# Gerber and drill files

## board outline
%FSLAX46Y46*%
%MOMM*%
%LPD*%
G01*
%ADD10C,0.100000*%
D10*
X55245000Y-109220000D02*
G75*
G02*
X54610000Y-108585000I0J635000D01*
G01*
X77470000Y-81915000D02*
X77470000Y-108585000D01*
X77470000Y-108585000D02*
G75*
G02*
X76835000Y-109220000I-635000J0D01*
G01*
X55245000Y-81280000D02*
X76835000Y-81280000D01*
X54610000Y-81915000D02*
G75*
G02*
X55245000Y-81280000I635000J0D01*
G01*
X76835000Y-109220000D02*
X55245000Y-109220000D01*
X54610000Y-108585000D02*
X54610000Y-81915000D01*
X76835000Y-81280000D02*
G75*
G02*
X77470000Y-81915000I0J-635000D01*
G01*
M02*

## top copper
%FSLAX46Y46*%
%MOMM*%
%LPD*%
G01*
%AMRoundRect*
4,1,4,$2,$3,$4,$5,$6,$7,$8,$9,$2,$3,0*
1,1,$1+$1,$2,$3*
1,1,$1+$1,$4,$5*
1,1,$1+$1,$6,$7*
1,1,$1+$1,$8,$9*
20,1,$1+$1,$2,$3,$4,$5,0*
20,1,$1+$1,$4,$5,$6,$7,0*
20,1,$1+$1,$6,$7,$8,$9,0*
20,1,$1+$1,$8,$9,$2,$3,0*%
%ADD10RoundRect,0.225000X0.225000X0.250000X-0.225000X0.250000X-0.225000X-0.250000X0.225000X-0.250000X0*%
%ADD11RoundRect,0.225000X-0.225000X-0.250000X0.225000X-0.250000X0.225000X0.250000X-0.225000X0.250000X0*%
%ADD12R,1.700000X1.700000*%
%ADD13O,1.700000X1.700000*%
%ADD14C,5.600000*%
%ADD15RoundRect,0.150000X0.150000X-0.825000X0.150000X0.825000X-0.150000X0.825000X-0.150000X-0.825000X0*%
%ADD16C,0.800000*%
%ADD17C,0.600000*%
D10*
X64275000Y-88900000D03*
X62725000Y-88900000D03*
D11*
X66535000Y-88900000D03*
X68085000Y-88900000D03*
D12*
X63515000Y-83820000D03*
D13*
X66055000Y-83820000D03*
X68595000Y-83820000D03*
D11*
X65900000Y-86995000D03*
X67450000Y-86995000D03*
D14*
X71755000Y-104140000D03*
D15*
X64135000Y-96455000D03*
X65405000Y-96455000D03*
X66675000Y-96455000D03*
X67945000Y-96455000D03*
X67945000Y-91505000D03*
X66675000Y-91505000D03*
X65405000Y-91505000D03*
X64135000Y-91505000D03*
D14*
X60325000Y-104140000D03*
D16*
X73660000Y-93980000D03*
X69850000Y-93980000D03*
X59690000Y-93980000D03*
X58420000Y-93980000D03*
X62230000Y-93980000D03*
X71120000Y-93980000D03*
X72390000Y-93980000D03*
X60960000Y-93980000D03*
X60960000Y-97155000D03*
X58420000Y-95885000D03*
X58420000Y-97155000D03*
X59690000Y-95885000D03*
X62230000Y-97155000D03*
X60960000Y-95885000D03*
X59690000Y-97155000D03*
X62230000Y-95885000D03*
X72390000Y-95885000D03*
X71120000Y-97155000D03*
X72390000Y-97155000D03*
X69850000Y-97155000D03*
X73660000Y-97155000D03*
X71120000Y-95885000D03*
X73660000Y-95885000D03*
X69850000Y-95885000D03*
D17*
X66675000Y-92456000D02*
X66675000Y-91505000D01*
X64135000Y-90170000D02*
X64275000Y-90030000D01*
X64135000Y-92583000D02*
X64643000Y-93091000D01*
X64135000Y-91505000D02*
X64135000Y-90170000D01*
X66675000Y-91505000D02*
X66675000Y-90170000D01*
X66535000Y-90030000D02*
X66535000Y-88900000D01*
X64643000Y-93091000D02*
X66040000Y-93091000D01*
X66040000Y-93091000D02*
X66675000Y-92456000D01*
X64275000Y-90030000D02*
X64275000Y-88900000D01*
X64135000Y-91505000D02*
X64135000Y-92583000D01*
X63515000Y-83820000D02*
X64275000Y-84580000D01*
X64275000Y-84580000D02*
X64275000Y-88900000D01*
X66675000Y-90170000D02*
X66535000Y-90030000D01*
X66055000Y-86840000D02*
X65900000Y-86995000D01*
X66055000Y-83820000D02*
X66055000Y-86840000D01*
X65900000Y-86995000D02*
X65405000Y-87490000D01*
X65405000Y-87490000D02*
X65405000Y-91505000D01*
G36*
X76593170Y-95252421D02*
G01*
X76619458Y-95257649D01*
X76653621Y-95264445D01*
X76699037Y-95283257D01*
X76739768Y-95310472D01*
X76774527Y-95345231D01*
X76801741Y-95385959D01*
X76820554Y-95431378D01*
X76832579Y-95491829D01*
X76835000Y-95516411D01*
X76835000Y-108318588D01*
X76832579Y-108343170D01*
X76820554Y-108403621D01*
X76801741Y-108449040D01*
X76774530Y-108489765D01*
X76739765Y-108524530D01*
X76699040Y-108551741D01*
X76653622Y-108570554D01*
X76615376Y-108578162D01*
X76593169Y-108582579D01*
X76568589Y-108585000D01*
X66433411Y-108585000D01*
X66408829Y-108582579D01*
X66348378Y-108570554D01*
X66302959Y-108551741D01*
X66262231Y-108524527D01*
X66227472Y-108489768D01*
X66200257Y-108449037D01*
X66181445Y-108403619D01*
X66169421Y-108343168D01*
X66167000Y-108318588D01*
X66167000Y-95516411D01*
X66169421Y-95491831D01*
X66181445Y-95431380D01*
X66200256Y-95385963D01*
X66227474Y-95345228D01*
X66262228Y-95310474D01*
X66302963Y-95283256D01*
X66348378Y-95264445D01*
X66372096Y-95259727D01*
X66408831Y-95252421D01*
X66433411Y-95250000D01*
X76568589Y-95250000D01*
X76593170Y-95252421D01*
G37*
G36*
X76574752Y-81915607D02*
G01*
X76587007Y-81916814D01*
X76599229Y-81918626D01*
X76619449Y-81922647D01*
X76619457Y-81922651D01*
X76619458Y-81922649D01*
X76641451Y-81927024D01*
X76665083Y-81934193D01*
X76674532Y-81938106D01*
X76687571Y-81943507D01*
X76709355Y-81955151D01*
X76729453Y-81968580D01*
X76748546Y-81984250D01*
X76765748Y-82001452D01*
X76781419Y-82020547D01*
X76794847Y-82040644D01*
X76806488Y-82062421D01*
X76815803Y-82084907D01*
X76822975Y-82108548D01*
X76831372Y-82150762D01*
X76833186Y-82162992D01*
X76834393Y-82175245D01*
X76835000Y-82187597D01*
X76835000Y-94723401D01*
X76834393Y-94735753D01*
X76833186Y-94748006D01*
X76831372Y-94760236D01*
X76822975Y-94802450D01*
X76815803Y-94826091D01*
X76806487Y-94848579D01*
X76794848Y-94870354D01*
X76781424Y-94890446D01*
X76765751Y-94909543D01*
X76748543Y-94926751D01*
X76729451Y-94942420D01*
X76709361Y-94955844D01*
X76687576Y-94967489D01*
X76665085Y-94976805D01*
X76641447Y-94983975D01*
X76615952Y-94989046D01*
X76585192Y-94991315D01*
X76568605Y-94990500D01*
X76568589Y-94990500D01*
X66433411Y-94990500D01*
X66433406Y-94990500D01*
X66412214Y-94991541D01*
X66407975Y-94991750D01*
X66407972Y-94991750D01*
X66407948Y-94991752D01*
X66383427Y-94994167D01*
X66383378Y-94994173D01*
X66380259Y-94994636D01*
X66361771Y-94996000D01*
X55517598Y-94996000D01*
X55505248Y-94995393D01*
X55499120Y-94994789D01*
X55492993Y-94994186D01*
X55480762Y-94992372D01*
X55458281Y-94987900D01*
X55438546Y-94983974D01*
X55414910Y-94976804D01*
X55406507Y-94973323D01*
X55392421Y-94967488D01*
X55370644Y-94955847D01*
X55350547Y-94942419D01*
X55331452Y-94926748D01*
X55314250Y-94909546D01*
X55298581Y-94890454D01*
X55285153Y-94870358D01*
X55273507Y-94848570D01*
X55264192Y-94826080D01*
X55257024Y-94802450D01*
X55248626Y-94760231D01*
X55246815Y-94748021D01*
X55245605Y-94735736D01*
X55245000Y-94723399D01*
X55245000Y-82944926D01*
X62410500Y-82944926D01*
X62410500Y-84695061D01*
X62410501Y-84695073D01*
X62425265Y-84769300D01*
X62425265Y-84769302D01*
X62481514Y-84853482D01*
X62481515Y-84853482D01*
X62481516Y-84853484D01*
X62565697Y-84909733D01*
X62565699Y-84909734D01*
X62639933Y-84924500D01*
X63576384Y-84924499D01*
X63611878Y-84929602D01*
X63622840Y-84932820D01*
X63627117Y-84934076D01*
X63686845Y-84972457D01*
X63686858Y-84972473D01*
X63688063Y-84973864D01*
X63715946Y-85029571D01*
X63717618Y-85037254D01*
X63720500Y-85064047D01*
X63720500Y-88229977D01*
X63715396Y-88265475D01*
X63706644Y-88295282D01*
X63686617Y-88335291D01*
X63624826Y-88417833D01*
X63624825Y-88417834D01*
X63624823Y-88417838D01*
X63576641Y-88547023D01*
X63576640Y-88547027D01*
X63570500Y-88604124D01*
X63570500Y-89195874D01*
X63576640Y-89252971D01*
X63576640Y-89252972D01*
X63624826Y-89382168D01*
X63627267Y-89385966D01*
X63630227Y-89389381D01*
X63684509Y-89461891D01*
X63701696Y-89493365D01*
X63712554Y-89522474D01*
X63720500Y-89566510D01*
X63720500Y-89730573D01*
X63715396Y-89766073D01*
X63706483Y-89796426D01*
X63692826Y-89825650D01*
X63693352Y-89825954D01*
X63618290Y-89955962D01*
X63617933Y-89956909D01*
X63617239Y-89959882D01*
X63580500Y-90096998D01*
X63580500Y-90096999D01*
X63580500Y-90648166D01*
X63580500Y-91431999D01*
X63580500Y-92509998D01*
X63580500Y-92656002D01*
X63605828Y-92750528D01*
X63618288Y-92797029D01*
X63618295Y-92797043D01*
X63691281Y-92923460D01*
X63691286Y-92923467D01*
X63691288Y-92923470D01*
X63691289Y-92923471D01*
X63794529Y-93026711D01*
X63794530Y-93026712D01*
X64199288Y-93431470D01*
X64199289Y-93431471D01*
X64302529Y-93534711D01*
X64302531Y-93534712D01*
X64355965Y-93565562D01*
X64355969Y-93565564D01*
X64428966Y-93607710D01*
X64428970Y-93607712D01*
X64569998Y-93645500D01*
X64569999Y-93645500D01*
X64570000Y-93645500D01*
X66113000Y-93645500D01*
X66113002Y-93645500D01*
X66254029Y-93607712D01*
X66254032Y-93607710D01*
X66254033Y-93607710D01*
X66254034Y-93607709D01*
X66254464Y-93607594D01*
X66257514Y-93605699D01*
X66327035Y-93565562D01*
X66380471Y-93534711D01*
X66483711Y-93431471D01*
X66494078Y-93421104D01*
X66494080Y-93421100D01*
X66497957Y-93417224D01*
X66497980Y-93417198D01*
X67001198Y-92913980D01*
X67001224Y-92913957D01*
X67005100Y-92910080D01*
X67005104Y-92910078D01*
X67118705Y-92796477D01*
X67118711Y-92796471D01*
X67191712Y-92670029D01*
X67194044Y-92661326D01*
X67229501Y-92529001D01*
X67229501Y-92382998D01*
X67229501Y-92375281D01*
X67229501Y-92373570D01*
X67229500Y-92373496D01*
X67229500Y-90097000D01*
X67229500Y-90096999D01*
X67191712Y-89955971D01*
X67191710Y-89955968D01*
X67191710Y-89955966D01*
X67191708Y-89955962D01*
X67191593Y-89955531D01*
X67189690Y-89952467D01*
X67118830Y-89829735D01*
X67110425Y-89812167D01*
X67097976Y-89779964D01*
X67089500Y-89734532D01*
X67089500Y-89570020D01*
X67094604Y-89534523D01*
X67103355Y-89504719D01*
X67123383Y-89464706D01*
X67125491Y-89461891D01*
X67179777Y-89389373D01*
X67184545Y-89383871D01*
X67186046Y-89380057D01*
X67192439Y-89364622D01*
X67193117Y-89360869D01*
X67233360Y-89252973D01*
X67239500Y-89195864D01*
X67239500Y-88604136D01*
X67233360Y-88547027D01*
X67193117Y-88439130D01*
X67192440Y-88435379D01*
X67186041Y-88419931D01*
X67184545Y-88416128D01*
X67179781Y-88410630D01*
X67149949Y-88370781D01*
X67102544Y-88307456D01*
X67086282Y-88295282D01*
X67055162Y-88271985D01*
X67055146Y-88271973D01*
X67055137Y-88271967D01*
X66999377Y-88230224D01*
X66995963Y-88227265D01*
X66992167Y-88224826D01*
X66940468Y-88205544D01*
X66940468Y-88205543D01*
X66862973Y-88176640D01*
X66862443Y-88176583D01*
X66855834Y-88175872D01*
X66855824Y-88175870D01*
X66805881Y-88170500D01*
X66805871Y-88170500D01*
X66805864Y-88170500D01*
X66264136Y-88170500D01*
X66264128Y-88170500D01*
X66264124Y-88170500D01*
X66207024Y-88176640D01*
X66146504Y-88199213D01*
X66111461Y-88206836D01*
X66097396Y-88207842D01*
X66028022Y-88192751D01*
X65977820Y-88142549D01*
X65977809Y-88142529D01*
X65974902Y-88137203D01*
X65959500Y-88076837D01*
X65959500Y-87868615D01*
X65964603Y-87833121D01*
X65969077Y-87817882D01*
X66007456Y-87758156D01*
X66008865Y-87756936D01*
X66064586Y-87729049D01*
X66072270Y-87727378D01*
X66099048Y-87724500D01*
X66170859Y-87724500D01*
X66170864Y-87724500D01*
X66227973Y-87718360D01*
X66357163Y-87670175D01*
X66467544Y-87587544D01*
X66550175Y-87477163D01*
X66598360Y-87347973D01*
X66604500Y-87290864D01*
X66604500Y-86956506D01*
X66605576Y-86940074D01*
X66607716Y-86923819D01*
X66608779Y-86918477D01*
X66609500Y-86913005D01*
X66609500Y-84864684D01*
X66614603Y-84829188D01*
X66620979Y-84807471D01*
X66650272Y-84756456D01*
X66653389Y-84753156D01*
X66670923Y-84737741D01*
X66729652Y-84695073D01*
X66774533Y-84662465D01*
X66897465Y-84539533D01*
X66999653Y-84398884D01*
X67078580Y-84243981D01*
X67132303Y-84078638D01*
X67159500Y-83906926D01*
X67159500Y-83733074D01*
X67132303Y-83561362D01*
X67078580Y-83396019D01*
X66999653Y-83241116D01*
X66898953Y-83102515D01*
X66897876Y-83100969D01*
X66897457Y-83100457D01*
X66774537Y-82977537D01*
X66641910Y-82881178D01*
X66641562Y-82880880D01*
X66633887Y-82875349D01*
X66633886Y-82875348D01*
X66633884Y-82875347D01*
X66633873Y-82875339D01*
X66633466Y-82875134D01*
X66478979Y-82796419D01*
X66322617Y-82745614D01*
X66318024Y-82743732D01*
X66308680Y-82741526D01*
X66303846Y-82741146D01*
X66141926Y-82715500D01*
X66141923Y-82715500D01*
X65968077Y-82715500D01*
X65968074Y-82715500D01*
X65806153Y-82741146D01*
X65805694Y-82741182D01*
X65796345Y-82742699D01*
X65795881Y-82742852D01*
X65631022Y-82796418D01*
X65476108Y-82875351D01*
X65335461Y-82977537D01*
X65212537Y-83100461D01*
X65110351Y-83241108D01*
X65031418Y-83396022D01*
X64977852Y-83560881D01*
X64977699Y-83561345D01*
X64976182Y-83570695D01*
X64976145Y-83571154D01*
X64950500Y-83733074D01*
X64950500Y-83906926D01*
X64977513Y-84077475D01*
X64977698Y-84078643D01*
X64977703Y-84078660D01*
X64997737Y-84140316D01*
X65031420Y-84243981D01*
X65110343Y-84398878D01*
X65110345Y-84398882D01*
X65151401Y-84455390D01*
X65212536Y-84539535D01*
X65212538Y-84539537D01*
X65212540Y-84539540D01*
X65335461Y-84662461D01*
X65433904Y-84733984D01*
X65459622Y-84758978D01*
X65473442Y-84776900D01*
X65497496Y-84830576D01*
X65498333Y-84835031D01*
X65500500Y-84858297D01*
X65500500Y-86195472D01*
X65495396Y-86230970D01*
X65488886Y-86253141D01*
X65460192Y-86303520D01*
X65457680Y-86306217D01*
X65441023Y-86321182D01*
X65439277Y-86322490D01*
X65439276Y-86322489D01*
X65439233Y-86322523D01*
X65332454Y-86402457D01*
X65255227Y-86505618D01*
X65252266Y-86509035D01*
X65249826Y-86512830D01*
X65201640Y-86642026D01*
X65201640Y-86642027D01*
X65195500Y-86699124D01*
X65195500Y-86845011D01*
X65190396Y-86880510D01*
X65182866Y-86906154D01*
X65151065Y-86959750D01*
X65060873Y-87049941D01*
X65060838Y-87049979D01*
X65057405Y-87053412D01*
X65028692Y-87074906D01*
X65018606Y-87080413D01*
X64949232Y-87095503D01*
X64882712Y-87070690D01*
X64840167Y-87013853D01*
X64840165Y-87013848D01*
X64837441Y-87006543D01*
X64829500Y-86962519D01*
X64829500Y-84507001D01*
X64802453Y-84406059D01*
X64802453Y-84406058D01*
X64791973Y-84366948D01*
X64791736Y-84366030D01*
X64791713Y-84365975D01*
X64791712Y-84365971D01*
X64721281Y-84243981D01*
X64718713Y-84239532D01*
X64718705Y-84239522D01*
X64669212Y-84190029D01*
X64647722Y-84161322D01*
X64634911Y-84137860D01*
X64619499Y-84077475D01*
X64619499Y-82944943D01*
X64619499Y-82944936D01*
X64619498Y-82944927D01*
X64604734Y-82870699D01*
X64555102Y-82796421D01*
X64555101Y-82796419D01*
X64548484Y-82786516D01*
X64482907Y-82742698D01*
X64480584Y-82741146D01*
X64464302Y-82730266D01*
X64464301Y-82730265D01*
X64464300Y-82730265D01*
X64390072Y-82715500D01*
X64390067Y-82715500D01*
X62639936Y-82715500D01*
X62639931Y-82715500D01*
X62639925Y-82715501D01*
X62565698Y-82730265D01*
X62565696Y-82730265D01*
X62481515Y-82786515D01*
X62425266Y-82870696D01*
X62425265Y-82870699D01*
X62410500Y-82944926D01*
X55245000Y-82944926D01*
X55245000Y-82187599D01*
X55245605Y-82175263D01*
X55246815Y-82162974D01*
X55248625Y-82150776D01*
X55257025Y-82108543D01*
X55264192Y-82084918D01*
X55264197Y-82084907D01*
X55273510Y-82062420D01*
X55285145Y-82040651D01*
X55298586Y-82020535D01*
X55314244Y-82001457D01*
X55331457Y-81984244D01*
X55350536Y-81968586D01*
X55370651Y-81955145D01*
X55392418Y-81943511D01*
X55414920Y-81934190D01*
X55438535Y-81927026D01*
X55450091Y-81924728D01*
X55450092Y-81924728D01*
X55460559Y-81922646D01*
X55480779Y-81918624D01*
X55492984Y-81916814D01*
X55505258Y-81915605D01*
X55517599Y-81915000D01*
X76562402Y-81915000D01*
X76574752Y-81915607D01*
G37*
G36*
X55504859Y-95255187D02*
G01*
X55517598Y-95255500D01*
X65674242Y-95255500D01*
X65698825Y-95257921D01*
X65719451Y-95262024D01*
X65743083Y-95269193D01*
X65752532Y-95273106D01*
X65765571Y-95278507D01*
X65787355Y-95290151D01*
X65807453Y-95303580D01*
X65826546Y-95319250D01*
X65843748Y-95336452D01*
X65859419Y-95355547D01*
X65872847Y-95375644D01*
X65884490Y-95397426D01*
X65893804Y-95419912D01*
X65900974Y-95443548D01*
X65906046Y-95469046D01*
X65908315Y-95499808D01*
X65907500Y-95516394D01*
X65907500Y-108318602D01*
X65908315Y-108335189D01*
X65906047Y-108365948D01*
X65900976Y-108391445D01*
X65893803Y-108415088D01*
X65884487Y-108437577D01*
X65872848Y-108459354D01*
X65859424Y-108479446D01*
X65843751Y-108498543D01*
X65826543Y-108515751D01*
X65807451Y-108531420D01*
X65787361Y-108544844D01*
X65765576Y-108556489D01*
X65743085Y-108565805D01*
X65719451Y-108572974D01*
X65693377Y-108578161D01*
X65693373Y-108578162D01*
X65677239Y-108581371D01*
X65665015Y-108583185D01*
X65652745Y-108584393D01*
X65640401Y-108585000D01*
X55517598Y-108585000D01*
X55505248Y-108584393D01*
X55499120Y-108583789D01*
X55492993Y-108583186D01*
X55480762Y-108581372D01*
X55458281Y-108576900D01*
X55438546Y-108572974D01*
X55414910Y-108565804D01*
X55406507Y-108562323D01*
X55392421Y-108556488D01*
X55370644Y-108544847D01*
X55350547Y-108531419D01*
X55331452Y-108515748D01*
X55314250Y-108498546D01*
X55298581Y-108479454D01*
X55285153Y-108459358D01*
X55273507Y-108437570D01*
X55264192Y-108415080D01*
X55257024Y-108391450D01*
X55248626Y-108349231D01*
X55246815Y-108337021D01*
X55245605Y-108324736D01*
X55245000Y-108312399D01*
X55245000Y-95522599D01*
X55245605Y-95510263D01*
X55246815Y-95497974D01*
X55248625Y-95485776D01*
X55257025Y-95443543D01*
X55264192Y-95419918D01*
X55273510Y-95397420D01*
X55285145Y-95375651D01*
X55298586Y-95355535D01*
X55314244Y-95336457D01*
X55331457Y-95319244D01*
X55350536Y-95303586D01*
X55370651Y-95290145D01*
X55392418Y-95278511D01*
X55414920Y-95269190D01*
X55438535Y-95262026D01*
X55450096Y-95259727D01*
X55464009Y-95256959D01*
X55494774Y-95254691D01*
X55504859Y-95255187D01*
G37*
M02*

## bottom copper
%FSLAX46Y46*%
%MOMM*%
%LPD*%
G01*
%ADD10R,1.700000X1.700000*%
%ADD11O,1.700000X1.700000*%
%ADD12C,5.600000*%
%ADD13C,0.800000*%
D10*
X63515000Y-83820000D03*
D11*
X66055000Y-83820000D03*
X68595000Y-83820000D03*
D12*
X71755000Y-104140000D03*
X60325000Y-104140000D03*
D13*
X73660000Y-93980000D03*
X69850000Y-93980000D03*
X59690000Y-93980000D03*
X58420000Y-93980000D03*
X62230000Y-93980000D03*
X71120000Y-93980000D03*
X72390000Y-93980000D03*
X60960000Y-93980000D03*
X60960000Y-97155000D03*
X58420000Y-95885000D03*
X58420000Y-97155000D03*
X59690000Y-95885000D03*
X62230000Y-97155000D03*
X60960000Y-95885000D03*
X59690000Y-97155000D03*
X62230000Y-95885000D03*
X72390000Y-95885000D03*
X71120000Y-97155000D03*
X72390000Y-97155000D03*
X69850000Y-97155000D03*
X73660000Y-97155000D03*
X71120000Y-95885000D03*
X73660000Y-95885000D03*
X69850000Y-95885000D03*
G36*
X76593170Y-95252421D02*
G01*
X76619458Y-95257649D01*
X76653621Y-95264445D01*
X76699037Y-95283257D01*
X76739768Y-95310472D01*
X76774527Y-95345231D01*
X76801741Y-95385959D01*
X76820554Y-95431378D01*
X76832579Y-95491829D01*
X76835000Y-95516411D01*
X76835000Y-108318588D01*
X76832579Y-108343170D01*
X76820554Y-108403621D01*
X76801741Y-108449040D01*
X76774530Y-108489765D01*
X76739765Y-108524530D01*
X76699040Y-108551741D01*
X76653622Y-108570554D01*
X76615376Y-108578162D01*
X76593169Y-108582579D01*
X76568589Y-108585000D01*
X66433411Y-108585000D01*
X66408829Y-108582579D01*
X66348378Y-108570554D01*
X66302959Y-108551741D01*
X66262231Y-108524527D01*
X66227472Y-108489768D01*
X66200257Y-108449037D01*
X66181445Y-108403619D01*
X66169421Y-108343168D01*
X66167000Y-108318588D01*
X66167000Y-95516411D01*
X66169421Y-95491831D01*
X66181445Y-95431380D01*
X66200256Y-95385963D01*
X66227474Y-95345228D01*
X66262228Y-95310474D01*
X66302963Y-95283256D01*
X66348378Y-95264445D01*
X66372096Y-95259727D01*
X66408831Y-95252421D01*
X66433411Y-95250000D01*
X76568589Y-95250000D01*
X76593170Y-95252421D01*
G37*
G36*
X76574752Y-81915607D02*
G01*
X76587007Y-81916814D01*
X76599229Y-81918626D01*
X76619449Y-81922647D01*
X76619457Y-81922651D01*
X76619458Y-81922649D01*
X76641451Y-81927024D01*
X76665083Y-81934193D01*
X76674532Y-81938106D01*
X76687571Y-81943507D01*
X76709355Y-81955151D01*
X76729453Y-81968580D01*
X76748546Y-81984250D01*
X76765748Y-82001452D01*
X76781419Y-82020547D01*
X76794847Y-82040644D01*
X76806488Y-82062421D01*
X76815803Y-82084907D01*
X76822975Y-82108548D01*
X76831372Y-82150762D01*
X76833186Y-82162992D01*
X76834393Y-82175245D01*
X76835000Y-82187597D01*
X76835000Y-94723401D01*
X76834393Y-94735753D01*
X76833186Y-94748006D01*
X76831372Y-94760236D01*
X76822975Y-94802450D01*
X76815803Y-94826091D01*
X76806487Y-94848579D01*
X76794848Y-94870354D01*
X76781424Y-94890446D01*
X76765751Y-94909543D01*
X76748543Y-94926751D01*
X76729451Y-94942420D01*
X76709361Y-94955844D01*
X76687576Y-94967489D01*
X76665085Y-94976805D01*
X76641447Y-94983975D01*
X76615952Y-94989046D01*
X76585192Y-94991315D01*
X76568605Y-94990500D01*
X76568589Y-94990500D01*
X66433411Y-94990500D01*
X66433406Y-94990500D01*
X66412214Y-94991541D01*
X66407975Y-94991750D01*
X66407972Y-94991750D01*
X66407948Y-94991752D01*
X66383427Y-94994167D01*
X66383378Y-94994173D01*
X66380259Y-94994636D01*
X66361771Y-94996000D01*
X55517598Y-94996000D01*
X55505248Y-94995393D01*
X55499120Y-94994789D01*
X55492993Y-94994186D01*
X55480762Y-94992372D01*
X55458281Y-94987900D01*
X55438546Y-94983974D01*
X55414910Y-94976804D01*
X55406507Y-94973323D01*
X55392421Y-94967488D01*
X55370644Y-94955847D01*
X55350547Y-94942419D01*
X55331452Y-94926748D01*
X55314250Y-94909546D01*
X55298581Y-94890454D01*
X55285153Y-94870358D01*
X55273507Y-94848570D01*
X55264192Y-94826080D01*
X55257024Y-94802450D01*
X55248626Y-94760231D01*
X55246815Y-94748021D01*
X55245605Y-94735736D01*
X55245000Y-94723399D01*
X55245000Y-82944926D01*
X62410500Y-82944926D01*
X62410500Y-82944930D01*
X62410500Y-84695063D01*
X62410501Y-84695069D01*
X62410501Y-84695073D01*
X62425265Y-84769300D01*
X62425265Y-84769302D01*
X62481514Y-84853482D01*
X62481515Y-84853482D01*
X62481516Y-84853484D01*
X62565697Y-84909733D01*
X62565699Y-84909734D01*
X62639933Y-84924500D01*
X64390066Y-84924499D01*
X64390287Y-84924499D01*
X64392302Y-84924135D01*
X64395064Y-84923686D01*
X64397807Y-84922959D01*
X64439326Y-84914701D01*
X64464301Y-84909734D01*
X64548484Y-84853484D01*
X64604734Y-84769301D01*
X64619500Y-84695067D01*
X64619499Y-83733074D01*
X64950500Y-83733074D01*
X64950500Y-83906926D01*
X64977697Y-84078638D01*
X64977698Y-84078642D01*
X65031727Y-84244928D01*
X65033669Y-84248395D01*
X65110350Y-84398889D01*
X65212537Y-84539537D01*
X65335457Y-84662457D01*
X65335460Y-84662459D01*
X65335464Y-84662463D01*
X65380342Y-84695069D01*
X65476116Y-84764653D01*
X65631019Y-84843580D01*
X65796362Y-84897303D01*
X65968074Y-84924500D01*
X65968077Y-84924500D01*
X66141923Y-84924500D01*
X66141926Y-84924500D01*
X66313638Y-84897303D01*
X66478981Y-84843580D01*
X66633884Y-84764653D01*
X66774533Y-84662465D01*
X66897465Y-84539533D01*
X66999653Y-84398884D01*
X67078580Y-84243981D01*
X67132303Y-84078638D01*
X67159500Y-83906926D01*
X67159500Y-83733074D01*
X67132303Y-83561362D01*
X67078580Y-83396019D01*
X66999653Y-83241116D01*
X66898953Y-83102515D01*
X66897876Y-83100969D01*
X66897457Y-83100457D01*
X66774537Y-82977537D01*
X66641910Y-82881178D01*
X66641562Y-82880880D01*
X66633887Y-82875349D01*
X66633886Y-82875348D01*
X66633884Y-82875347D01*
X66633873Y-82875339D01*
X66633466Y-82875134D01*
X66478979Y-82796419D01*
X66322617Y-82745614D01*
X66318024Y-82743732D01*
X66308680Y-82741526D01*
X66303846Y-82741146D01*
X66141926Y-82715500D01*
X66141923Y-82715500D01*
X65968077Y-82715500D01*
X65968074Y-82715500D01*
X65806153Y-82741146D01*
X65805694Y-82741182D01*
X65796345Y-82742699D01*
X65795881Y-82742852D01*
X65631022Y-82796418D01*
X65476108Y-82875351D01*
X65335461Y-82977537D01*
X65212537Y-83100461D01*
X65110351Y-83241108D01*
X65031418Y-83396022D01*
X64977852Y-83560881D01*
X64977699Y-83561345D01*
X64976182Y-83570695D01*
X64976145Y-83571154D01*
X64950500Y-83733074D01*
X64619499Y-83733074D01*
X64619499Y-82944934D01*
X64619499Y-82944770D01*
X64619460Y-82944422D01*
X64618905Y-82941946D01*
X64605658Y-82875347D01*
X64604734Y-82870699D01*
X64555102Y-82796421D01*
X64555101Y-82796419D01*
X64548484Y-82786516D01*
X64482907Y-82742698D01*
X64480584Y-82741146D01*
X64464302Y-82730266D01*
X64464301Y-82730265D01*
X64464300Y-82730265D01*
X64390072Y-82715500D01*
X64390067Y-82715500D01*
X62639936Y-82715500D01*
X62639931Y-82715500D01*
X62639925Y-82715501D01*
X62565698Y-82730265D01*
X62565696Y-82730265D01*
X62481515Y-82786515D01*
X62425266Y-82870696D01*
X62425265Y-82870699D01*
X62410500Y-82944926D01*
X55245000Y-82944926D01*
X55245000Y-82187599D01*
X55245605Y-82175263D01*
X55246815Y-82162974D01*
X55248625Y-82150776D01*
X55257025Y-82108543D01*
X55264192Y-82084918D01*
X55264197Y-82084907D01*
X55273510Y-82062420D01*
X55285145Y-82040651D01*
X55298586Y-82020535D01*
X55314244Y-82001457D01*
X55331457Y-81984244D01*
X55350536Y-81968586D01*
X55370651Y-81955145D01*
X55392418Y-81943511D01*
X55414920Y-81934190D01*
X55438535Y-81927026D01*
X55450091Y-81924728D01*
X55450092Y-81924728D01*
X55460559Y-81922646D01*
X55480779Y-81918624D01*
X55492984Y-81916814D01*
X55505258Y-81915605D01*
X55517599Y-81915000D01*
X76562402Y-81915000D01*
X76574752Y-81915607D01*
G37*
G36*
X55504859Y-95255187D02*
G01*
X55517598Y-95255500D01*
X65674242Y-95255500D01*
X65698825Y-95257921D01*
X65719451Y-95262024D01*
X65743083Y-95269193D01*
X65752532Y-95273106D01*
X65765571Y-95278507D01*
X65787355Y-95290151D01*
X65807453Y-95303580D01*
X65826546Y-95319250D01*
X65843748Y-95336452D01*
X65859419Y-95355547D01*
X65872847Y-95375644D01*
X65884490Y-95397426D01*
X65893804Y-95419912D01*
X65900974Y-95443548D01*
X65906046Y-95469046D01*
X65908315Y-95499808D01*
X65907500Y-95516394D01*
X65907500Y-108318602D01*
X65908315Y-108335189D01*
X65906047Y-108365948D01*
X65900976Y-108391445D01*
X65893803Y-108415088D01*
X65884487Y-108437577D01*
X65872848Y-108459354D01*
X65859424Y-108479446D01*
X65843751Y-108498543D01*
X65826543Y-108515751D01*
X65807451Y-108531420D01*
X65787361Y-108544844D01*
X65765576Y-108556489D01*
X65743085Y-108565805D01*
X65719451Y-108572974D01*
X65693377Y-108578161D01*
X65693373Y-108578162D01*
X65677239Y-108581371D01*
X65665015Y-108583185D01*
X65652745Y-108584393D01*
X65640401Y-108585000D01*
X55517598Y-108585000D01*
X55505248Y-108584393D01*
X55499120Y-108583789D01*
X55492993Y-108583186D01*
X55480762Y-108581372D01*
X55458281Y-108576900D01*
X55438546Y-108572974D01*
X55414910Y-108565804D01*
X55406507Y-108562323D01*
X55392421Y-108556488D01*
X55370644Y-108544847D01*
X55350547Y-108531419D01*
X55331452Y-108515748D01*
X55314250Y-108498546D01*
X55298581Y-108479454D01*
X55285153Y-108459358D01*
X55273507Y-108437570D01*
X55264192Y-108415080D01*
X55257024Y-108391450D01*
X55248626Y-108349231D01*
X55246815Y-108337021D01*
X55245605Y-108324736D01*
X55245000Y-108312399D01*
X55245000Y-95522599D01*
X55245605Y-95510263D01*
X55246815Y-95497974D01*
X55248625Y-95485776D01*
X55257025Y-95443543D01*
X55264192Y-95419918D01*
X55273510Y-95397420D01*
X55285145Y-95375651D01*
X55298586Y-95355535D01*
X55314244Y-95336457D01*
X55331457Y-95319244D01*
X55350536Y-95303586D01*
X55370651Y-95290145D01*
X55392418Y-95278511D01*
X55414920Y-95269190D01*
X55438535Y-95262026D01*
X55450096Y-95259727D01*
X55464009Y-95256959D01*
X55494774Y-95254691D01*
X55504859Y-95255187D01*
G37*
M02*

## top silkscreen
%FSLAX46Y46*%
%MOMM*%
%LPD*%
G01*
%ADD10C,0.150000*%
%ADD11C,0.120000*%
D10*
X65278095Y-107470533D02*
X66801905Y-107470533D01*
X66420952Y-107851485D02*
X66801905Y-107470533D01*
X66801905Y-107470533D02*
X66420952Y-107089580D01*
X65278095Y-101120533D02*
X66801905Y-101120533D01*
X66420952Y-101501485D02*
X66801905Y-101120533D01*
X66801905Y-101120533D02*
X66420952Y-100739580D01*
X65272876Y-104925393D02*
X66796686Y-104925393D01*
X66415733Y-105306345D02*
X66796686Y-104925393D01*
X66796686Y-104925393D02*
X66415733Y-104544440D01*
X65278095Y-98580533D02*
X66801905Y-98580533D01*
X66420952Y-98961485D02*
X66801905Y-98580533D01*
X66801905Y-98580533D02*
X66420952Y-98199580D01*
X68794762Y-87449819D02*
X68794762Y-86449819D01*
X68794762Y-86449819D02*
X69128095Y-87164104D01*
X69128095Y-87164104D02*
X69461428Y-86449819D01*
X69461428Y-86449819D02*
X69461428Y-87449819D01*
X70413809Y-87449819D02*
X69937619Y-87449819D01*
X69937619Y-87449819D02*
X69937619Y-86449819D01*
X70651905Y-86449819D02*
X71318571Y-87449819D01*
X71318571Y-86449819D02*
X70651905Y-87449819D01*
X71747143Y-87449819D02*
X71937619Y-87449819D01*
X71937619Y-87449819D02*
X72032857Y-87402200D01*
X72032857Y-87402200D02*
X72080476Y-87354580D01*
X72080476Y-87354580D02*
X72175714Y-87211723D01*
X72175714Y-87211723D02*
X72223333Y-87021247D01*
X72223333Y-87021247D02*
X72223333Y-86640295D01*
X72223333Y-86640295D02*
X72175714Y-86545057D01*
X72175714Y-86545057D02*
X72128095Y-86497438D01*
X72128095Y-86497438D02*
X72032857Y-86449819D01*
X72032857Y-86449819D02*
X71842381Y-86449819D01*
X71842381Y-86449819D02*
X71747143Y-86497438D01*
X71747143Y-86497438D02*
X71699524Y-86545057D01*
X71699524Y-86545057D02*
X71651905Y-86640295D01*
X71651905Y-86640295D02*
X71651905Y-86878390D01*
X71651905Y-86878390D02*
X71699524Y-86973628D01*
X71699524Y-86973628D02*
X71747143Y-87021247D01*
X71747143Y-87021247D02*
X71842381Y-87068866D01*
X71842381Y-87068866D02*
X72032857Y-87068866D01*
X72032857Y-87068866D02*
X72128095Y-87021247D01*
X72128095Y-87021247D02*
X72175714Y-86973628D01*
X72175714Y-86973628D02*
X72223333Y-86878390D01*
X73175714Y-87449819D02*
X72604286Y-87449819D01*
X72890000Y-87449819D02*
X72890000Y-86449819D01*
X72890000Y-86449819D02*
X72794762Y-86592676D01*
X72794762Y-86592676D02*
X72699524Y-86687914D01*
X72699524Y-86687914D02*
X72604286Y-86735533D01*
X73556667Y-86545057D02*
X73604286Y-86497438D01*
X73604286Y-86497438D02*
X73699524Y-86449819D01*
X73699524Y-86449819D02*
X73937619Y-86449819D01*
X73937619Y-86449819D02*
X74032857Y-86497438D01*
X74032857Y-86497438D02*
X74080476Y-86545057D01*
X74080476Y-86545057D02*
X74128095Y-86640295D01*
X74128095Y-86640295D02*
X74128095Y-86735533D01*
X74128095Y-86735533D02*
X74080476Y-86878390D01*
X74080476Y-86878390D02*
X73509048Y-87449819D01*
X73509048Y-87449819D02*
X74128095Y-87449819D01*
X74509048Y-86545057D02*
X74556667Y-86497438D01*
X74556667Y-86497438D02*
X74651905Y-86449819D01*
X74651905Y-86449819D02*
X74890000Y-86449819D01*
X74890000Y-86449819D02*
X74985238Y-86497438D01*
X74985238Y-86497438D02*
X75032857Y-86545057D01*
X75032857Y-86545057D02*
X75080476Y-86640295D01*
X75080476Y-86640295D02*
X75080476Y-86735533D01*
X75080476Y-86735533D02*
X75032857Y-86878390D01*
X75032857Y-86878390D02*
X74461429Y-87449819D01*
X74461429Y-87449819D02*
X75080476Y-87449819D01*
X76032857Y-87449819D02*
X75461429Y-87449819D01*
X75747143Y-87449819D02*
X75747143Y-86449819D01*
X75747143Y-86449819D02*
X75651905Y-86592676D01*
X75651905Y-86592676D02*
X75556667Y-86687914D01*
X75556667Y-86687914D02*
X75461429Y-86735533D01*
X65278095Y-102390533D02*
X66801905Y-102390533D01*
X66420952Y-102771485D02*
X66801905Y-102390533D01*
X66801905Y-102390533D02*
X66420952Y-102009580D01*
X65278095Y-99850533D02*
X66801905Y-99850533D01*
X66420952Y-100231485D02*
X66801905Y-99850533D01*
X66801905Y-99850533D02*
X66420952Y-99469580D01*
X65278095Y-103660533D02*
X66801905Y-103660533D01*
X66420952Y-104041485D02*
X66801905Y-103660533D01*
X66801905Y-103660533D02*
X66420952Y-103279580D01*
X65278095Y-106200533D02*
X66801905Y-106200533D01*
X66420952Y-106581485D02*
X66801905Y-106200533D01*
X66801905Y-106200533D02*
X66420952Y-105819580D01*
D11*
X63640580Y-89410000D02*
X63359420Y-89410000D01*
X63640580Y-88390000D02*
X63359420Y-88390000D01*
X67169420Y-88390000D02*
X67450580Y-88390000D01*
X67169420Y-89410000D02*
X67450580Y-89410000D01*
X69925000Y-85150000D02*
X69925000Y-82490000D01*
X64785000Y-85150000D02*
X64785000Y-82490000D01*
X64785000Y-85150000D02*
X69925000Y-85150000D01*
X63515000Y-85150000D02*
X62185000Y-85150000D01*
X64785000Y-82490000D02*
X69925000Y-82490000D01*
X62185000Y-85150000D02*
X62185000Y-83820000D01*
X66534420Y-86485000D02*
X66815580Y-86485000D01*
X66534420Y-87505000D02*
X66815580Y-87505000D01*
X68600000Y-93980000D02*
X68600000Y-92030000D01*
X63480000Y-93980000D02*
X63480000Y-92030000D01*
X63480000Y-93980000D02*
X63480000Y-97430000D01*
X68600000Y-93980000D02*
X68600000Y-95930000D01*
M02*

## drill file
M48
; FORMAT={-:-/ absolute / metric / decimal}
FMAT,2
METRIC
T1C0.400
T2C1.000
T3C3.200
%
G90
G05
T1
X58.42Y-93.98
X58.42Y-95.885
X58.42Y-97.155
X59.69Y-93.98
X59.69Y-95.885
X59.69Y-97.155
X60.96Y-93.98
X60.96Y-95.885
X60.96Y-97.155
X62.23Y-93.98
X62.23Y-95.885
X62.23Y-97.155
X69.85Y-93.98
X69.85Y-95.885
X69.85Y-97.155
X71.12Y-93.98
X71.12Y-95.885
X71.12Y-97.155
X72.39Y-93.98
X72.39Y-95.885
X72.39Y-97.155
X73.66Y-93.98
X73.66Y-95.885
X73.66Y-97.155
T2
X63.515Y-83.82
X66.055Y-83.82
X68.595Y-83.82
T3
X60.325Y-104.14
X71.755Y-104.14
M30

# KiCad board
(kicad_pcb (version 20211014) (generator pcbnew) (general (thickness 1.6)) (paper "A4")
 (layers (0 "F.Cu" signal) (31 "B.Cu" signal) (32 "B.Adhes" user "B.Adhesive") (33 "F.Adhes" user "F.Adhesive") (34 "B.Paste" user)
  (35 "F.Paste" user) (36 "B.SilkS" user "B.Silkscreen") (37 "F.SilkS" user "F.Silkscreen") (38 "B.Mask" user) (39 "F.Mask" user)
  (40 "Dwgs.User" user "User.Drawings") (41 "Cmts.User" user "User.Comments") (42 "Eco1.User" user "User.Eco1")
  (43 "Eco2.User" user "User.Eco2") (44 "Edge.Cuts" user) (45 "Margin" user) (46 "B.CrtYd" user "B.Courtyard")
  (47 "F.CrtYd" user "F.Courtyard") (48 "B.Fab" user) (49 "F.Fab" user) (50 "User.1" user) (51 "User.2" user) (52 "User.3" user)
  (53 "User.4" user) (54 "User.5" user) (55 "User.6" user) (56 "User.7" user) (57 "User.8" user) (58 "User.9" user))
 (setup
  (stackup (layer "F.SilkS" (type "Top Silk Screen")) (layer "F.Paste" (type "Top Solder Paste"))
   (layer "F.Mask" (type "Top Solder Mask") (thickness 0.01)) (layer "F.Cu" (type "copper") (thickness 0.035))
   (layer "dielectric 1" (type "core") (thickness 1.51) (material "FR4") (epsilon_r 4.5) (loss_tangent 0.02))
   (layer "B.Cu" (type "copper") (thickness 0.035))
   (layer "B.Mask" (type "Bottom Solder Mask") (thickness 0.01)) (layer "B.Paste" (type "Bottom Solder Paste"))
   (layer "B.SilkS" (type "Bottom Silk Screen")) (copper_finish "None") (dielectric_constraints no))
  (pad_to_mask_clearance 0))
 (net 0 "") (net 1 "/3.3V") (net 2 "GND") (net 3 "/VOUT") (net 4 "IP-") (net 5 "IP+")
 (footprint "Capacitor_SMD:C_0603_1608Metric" (layer "F.Cu") (at 63.5 88.9 180)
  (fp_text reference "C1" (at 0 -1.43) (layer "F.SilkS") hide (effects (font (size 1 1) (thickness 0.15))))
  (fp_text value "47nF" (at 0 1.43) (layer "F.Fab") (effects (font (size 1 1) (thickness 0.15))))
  (fp_line (start -0.14058 -0.51) (end 0.14058 -0.51) (layer "F.SilkS") (width 0.12))
  (fp_line (start -0.14058 0.51) (end 0.14058 0.51) (layer "F.SilkS") (width 0.12))
  (pad "1" smd roundrect (at -0.775 0 180) (size 0.9 0.95) (layers "F.Cu" "F.Paste" "F.Mask") (roundrect_rratio 0.25) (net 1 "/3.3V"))
  (pad "2" smd roundrect (at 0.775 0 180) (size 0.9 0.95) (layers "F.Cu" "F.Paste" "F.Mask") (roundrect_rratio 0.25) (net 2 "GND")))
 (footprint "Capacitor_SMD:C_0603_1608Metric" (layer "F.Cu") (at 67.31 88.9)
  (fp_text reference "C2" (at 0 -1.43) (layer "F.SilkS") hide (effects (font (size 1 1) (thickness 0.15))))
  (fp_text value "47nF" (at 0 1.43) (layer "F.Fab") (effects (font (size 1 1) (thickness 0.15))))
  (fp_line (start -0.14058 -0.51) (end 0.14058 -0.51) (layer "F.SilkS") (width 0.12))
  (fp_line (start -0.14058 0.51) (end 0.14058 0.51) (layer "F.SilkS") (width 0.12))
  (pad "1" smd roundrect (at -0.775 0) (size 0.9 0.95) (layers "F.Cu" "F.Paste" "F.Mask") (roundrect_rratio 0.25) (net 1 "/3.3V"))
  (pad "2" smd roundrect (at 0.775 0) (size 0.9 0.95) (layers "F.Cu" "F.Paste" "F.Mask") (roundrect_rratio 0.25) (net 2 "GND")))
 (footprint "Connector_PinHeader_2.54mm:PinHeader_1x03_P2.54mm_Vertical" (layer "F.Cu") (at 63.515 83.82 90)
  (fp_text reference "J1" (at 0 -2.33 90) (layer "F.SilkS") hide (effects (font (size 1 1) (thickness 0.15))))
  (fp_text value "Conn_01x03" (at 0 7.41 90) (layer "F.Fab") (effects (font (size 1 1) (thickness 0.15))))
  (fp_line (start -1.33 6.41) (end 1.33 6.41) (layer "F.SilkS") (width 0.12))
  (fp_line (start -1.33 1.27) (end 1.33 1.27) (layer "F.SilkS") (width 0.12))
  (fp_line (start -1.33 1.27) (end -1.33 6.41) (layer "F.SilkS") (width 0.12))
  (fp_line (start -1.33 0) (end -1.33 -1.33) (layer "F.SilkS") (width 0.12))
  (fp_line (start 1.33 1.27) (end 1.33 6.41) (layer "F.SilkS") (width 0.12))
  (fp_line (start -1.33 -1.33) (end 0 -1.33) (layer "F.SilkS") (width 0.12))
  (pad "1" thru_hole rect (at 0 0 90) (size 1.7 1.7) (drill 1) (layers *.Cu *.Mask) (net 1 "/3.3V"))
  (pad "2" thru_hole oval (at 0 2.54 90) (size 1.7 1.7) (drill 1) (layers *.Cu *.Mask) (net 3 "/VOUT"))
  (pad "3" thru_hole oval (at 0 5.08 90) (size 1.7 1.7) (drill 1) (layers *.Cu *.Mask) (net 2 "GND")))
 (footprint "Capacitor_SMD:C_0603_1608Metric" (layer "F.Cu") (at 66.675 86.995)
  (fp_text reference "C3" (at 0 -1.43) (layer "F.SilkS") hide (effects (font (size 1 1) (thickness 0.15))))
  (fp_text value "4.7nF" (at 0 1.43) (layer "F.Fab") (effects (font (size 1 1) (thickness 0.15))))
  (fp_line (start -0.14058 -0.51) (end 0.14058 -0.51) (layer "F.SilkS") (width 0.12))
  (fp_line (start -0.14058 0.51) (end 0.14058 0.51) (layer "F.SilkS") (width 0.12))
  (pad "1" smd roundrect (at -0.775 0) (size 0.9 0.95) (layers "F.Cu" "F.Paste" "F.Mask") (roundrect_rratio 0.25) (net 3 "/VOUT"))
  (pad "2" smd roundrect (at 0.775 0) (size 0.9 0.95) (layers "F.Cu" "F.Paste" "F.Mask") (roundrect_rratio 0.25) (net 2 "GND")))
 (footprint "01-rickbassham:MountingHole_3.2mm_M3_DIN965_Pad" (layer "F.Cu") (at 71.755 104.14)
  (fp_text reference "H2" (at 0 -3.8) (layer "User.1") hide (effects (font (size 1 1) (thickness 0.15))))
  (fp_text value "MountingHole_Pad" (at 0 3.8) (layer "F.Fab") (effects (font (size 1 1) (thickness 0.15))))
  (pad "1" thru_hole circle (at 0 0) (size 5.6 5.6) (drill 3.2) (layers *.Cu *.Mask) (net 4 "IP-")))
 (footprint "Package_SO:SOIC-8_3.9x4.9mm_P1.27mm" (layer "F.Cu") (at 66.04 93.98 90)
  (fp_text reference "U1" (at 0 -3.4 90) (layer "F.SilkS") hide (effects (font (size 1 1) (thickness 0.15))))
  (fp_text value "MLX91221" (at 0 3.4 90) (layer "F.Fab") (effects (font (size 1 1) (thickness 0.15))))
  (fp_line (start 0 2.56) (end 1.95 2.56) (layer "F.SilkS") (width 0.12))
  (fp_line (start 0 -2.56) (end 1.95 -2.56) (layer "F.SilkS") (width 0.12))
  (fp_line (start 0 -2.56) (end -3.45 -2.56) (layer "F.SilkS") (width 0.12))
  (fp_line (start 0 2.56) (end -1.95 2.56) (layer "F.SilkS") (width 0.12))
  (pad "1" smd roundrect (at -2.475 -1.905 90) (size 1.95 0.6) (layers "F.Cu" "F.Paste" "F.Mask") (roundrect_rratio 0.25) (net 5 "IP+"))
  (pad "2" smd roundrect (at -2.475 -0.635 90) (size 1.95 0.6) (layers "F.Cu" "F.Paste" "F.Mask") (roundrect_rratio 0.25) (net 5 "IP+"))
  (pad "3" smd roundrect (at -2.475 0.635 90) (size 1.95 0.6) (layers "F.Cu" "F.Paste" "F.Mask") (roundrect_rratio 0.25) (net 4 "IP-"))
  (pad "4" smd roundrect (at -2.475 1.905 90) (size 1.95 0.6) (layers "F.Cu" "F.Paste" "F.Mask") (roundrect_rratio 0.25) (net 4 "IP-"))
  (pad "5" smd roundrect (at 2.475 1.905 90) (size 1.95 0.6) (layers "F.Cu" "F.Paste" "F.Mask") (roundrect_rratio 0.25) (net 2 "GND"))
  (pad "6" smd roundrect (at 2.475 0.635 90) (size 1.95 0.6) (layers "F.Cu" "F.Paste" "F.Mask") (roundrect_rratio 0.25) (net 1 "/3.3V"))
  (pad "7" smd roundrect (at 2.475 -0.635 90) (size 1.95 0.6) (layers "F.Cu" "F.Paste" "F.Mask") (roundrect_rratio 0.25) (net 3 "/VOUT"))
  (pad "8" smd roundrect (at 2.475 -1.905 90) (size 1.95 0.6) (layers "F.Cu" "F.Paste" "F.Mask") (roundrect_rratio 0.25) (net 1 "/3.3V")))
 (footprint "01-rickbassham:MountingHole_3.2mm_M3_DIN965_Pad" (layer "F.Cu") (at 60.325 104.14)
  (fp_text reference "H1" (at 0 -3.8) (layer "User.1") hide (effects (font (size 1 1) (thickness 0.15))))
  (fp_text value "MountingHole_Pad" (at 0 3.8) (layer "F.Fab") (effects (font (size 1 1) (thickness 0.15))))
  (pad "1" thru_hole circle (at 0 0) (size 5.6 5.6) (drill 3.2) (layers *.Cu *.Mask) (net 5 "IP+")))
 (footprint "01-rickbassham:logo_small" (layer "B.Cu") (at 66.04 93.98 180)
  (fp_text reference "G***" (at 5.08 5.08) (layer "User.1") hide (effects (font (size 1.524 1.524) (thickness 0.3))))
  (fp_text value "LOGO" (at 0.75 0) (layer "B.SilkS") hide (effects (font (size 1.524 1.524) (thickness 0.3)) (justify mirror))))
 (gr_arc (start 55.245 109.22) (mid 54.795987 109.034013) (end 54.61 108.585) (layer "Edge.Cuts") (width 0.1))
 (gr_line (start 77.47 81.915) (end 77.47 108.585) (layer "Edge.Cuts") (width 0.1))
 (gr_arc (start 77.47 108.585) (mid 77.284013 109.034013) (end 76.835 109.22) (layer "Edge.Cuts") (width 0.1))
 (gr_line (start 55.245 81.28) (end 76.835 81.28) (layer "Edge.Cuts") (width 0.1))
 (gr_arc (start 54.61 81.915) (mid 54.795987 81.465987) (end 55.245 81.28) (layer "Edge.Cuts") (width 0.1))
 (gr_line (start 76.835 109.22) (end 55.245 109.22) (layer "Edge.Cuts") (width 0.1))
 (gr_line (start 54.61 108.585) (end 54.61 81.915) (layer "Edge.Cuts") (width 0.1))
 (gr_arc (start 76.835 81.28) (mid 77.284013 81.465987) (end 77.47 81.915) (layer "Edge.Cuts") (width 0.1))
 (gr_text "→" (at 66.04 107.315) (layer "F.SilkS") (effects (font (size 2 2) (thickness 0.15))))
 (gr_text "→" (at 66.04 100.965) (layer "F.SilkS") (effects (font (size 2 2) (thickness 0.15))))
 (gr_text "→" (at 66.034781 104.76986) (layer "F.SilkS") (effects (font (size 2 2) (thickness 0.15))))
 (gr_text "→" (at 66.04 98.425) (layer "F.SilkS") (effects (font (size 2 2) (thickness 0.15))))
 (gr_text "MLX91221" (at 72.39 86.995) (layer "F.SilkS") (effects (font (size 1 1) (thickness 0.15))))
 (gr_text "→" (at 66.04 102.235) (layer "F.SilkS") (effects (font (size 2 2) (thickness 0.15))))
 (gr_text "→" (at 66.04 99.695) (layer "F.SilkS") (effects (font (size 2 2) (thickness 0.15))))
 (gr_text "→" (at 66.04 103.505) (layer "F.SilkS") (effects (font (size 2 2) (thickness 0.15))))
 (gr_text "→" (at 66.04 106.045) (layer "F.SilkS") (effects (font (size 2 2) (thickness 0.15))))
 (segment (start 66.675 92.456) (end 66.675 91.505) (width 0.6) (layer "F.Cu") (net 1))
 (segment (start 64.135 90.17) (end 64.275 90.03) (width 0.6) (layer "F.Cu") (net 1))
 (segment (start 64.135 92.583) (end 64.643 93.091) (width 0.6) (layer "F.Cu") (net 1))
 (segment (start 64.135 91.505) (end 64.135 90.17) (width 0.6) (layer "F.Cu") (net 1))
 (segment (start 66.675 91.505) (end 66.675 90.17) (width 0.6) (layer "F.Cu") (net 1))
 (segment (start 66.535 90.03) (end 66.535 88.9) (width 0.6) (layer "F.Cu") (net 1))
 (segment (start 64.643 93.091) (end 66.04 93.091) (width 0.6) (layer "F.Cu") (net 1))
 (segment (start 66.04 93.091) (end 66.675 92.456) (width 0.6) (layer "F.Cu") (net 1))
 (segment (start 64.275 90.03) (end 64.275 88.9) (width 0.6) (layer "F.Cu") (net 1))
 (segment (start 64.135 91.505) (end 64.135 92.583) (width 0.6) (layer "F.Cu") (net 1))
 (segment (start 63.515 83.82) (end 64.275 84.58) (width 0.6) (layer "F.Cu") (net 1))
 (segment (start 64.275 84.58) (end 64.275 88.9) (width 0.6) (layer "F.Cu") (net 1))
 (segment (start 66.675 90.17) (end 66.535 90.03) (width 0.6) (layer "F.Cu") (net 1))
 (via (at 73.66 93.98) (size 0.8) (drill 0.4) (layers "F.Cu" "B.Cu") (free) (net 2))
 (via (at 69.85 93.98) (size 0.8) (drill 0.4) (layers "F.Cu" "B.Cu") (free) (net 2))
 (via (at 59.69 93.98) (size 0.8) (drill 0.4) (layers "F.Cu" "B.Cu") (free) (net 2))
 (via (at 58.42 93.98) (size 0.8) (drill 0.4) (layers "F.Cu" "B.Cu") (free) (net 2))
 (via (at 62.23 93.98) (size 0.8) (drill 0.4) (layers "F.Cu" "B.Cu") (free) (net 2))
 (via (at 71.12 93.98) (size 0.8) (drill 0.4) (layers "F.Cu" "B.Cu") (free) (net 2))
 (via (at 72.39 93.98) (size 0.8) (drill 0.4) (layers "F.Cu" "B.Cu") (free) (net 2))
 (via (at 60.96 93.98) (size 0.8) (drill 0.4) (layers "F.Cu" "B.Cu") (free) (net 2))
 (segment (start 66.055 86.84) (end 65.9 86.995) (width 0.6) (layer "F.Cu") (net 3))
 (segment (start 66.055 83.82) (end 66.055 86.84) (width 0.6) (layer "F.Cu") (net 3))
 (segment (start 65.9 86.995) (end 65.405 87.49) (width 0.6) (layer "F.Cu") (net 3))
 (segment (start 65.405 87.49) (end 65.405 91.505) (width 0.6) (layer "F.Cu") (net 3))
 (via (at 60.96 97.155) (size 0.8) (drill 0.4) (layers "F.Cu" "B.Cu") (free) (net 5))
 (via (at 58.42 95.885) (size 0.8) (drill 0.4) (layers "F.Cu" "B.Cu") (free) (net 5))
 (via (at 58.42 97.155) (size 0.8) (drill 0.4) (layers "F.Cu" "B.Cu") (free) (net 5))
 (via (at 59.69 95.885) (size 0.8) (drill 0.4) (layers "F.Cu" "B.Cu") (free) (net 5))
 (via (at 62.23 97.155) (size 0.8) (drill 0.4) (layers "F.Cu" "B.Cu") (free) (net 5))
 (via (at 60.96 95.885) (size 0.8) (drill 0.4) (layers "F.Cu" "B.Cu") (free) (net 5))
 (via (at 59.69 97.155) (size 0.8) (drill 0.4) (layers "F.Cu" "B.Cu") (free) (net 5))
 (via (at 62.23 95.885) (size 0.8) (drill 0.4) (layers "F.Cu" "B.Cu") (free) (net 5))
 (via (at 72.39 95.885) (size 0.8) (drill 0.4) (layers "F.Cu" "B.Cu") (free) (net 4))
 (via (at 71.12 97.155) (size 0.8) (drill 0.4) (layers "F.Cu" "B.Cu") (free) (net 4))
 (via (at 72.39 97.155) (size 0.8) (drill 0.4) (layers "F.Cu" "B.Cu") (free) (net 4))
 (via (at 69.85 97.155) (size 0.8) (drill 0.4) (layers "F.Cu" "B.Cu") (free) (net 4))
 (via (at 73.66 97.155) (size 0.8) (drill 0.4) (layers "F.Cu" "B.Cu") (free) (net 4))
 (via (at 71.12 95.885) (size 0.8) (drill 0.4) (layers "F.Cu" "B.Cu") (free) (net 4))
 (via (at 73.66 95.885) (size 0.8) (drill 0.4) (layers "F.Cu" "B.Cu") (free) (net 4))
 (via (at 69.85 95.885) (size 0.8) (drill 0.4) (layers "F.Cu" "B.Cu") (free) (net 4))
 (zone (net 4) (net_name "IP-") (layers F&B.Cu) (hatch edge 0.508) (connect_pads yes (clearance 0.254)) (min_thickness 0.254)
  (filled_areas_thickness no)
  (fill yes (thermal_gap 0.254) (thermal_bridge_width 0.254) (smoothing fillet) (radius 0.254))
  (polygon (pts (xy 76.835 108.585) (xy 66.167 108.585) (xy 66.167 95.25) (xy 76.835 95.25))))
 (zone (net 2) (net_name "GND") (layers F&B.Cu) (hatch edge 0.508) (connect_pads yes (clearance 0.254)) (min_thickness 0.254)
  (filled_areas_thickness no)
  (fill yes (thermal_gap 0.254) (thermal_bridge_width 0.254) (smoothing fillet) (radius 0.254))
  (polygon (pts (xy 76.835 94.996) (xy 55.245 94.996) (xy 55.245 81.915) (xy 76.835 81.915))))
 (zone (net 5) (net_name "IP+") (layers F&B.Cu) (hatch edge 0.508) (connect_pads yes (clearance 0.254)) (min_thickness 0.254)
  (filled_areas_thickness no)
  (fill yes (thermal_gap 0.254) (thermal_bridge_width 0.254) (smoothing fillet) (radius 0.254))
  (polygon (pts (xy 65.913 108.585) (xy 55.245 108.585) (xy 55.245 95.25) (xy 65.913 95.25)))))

